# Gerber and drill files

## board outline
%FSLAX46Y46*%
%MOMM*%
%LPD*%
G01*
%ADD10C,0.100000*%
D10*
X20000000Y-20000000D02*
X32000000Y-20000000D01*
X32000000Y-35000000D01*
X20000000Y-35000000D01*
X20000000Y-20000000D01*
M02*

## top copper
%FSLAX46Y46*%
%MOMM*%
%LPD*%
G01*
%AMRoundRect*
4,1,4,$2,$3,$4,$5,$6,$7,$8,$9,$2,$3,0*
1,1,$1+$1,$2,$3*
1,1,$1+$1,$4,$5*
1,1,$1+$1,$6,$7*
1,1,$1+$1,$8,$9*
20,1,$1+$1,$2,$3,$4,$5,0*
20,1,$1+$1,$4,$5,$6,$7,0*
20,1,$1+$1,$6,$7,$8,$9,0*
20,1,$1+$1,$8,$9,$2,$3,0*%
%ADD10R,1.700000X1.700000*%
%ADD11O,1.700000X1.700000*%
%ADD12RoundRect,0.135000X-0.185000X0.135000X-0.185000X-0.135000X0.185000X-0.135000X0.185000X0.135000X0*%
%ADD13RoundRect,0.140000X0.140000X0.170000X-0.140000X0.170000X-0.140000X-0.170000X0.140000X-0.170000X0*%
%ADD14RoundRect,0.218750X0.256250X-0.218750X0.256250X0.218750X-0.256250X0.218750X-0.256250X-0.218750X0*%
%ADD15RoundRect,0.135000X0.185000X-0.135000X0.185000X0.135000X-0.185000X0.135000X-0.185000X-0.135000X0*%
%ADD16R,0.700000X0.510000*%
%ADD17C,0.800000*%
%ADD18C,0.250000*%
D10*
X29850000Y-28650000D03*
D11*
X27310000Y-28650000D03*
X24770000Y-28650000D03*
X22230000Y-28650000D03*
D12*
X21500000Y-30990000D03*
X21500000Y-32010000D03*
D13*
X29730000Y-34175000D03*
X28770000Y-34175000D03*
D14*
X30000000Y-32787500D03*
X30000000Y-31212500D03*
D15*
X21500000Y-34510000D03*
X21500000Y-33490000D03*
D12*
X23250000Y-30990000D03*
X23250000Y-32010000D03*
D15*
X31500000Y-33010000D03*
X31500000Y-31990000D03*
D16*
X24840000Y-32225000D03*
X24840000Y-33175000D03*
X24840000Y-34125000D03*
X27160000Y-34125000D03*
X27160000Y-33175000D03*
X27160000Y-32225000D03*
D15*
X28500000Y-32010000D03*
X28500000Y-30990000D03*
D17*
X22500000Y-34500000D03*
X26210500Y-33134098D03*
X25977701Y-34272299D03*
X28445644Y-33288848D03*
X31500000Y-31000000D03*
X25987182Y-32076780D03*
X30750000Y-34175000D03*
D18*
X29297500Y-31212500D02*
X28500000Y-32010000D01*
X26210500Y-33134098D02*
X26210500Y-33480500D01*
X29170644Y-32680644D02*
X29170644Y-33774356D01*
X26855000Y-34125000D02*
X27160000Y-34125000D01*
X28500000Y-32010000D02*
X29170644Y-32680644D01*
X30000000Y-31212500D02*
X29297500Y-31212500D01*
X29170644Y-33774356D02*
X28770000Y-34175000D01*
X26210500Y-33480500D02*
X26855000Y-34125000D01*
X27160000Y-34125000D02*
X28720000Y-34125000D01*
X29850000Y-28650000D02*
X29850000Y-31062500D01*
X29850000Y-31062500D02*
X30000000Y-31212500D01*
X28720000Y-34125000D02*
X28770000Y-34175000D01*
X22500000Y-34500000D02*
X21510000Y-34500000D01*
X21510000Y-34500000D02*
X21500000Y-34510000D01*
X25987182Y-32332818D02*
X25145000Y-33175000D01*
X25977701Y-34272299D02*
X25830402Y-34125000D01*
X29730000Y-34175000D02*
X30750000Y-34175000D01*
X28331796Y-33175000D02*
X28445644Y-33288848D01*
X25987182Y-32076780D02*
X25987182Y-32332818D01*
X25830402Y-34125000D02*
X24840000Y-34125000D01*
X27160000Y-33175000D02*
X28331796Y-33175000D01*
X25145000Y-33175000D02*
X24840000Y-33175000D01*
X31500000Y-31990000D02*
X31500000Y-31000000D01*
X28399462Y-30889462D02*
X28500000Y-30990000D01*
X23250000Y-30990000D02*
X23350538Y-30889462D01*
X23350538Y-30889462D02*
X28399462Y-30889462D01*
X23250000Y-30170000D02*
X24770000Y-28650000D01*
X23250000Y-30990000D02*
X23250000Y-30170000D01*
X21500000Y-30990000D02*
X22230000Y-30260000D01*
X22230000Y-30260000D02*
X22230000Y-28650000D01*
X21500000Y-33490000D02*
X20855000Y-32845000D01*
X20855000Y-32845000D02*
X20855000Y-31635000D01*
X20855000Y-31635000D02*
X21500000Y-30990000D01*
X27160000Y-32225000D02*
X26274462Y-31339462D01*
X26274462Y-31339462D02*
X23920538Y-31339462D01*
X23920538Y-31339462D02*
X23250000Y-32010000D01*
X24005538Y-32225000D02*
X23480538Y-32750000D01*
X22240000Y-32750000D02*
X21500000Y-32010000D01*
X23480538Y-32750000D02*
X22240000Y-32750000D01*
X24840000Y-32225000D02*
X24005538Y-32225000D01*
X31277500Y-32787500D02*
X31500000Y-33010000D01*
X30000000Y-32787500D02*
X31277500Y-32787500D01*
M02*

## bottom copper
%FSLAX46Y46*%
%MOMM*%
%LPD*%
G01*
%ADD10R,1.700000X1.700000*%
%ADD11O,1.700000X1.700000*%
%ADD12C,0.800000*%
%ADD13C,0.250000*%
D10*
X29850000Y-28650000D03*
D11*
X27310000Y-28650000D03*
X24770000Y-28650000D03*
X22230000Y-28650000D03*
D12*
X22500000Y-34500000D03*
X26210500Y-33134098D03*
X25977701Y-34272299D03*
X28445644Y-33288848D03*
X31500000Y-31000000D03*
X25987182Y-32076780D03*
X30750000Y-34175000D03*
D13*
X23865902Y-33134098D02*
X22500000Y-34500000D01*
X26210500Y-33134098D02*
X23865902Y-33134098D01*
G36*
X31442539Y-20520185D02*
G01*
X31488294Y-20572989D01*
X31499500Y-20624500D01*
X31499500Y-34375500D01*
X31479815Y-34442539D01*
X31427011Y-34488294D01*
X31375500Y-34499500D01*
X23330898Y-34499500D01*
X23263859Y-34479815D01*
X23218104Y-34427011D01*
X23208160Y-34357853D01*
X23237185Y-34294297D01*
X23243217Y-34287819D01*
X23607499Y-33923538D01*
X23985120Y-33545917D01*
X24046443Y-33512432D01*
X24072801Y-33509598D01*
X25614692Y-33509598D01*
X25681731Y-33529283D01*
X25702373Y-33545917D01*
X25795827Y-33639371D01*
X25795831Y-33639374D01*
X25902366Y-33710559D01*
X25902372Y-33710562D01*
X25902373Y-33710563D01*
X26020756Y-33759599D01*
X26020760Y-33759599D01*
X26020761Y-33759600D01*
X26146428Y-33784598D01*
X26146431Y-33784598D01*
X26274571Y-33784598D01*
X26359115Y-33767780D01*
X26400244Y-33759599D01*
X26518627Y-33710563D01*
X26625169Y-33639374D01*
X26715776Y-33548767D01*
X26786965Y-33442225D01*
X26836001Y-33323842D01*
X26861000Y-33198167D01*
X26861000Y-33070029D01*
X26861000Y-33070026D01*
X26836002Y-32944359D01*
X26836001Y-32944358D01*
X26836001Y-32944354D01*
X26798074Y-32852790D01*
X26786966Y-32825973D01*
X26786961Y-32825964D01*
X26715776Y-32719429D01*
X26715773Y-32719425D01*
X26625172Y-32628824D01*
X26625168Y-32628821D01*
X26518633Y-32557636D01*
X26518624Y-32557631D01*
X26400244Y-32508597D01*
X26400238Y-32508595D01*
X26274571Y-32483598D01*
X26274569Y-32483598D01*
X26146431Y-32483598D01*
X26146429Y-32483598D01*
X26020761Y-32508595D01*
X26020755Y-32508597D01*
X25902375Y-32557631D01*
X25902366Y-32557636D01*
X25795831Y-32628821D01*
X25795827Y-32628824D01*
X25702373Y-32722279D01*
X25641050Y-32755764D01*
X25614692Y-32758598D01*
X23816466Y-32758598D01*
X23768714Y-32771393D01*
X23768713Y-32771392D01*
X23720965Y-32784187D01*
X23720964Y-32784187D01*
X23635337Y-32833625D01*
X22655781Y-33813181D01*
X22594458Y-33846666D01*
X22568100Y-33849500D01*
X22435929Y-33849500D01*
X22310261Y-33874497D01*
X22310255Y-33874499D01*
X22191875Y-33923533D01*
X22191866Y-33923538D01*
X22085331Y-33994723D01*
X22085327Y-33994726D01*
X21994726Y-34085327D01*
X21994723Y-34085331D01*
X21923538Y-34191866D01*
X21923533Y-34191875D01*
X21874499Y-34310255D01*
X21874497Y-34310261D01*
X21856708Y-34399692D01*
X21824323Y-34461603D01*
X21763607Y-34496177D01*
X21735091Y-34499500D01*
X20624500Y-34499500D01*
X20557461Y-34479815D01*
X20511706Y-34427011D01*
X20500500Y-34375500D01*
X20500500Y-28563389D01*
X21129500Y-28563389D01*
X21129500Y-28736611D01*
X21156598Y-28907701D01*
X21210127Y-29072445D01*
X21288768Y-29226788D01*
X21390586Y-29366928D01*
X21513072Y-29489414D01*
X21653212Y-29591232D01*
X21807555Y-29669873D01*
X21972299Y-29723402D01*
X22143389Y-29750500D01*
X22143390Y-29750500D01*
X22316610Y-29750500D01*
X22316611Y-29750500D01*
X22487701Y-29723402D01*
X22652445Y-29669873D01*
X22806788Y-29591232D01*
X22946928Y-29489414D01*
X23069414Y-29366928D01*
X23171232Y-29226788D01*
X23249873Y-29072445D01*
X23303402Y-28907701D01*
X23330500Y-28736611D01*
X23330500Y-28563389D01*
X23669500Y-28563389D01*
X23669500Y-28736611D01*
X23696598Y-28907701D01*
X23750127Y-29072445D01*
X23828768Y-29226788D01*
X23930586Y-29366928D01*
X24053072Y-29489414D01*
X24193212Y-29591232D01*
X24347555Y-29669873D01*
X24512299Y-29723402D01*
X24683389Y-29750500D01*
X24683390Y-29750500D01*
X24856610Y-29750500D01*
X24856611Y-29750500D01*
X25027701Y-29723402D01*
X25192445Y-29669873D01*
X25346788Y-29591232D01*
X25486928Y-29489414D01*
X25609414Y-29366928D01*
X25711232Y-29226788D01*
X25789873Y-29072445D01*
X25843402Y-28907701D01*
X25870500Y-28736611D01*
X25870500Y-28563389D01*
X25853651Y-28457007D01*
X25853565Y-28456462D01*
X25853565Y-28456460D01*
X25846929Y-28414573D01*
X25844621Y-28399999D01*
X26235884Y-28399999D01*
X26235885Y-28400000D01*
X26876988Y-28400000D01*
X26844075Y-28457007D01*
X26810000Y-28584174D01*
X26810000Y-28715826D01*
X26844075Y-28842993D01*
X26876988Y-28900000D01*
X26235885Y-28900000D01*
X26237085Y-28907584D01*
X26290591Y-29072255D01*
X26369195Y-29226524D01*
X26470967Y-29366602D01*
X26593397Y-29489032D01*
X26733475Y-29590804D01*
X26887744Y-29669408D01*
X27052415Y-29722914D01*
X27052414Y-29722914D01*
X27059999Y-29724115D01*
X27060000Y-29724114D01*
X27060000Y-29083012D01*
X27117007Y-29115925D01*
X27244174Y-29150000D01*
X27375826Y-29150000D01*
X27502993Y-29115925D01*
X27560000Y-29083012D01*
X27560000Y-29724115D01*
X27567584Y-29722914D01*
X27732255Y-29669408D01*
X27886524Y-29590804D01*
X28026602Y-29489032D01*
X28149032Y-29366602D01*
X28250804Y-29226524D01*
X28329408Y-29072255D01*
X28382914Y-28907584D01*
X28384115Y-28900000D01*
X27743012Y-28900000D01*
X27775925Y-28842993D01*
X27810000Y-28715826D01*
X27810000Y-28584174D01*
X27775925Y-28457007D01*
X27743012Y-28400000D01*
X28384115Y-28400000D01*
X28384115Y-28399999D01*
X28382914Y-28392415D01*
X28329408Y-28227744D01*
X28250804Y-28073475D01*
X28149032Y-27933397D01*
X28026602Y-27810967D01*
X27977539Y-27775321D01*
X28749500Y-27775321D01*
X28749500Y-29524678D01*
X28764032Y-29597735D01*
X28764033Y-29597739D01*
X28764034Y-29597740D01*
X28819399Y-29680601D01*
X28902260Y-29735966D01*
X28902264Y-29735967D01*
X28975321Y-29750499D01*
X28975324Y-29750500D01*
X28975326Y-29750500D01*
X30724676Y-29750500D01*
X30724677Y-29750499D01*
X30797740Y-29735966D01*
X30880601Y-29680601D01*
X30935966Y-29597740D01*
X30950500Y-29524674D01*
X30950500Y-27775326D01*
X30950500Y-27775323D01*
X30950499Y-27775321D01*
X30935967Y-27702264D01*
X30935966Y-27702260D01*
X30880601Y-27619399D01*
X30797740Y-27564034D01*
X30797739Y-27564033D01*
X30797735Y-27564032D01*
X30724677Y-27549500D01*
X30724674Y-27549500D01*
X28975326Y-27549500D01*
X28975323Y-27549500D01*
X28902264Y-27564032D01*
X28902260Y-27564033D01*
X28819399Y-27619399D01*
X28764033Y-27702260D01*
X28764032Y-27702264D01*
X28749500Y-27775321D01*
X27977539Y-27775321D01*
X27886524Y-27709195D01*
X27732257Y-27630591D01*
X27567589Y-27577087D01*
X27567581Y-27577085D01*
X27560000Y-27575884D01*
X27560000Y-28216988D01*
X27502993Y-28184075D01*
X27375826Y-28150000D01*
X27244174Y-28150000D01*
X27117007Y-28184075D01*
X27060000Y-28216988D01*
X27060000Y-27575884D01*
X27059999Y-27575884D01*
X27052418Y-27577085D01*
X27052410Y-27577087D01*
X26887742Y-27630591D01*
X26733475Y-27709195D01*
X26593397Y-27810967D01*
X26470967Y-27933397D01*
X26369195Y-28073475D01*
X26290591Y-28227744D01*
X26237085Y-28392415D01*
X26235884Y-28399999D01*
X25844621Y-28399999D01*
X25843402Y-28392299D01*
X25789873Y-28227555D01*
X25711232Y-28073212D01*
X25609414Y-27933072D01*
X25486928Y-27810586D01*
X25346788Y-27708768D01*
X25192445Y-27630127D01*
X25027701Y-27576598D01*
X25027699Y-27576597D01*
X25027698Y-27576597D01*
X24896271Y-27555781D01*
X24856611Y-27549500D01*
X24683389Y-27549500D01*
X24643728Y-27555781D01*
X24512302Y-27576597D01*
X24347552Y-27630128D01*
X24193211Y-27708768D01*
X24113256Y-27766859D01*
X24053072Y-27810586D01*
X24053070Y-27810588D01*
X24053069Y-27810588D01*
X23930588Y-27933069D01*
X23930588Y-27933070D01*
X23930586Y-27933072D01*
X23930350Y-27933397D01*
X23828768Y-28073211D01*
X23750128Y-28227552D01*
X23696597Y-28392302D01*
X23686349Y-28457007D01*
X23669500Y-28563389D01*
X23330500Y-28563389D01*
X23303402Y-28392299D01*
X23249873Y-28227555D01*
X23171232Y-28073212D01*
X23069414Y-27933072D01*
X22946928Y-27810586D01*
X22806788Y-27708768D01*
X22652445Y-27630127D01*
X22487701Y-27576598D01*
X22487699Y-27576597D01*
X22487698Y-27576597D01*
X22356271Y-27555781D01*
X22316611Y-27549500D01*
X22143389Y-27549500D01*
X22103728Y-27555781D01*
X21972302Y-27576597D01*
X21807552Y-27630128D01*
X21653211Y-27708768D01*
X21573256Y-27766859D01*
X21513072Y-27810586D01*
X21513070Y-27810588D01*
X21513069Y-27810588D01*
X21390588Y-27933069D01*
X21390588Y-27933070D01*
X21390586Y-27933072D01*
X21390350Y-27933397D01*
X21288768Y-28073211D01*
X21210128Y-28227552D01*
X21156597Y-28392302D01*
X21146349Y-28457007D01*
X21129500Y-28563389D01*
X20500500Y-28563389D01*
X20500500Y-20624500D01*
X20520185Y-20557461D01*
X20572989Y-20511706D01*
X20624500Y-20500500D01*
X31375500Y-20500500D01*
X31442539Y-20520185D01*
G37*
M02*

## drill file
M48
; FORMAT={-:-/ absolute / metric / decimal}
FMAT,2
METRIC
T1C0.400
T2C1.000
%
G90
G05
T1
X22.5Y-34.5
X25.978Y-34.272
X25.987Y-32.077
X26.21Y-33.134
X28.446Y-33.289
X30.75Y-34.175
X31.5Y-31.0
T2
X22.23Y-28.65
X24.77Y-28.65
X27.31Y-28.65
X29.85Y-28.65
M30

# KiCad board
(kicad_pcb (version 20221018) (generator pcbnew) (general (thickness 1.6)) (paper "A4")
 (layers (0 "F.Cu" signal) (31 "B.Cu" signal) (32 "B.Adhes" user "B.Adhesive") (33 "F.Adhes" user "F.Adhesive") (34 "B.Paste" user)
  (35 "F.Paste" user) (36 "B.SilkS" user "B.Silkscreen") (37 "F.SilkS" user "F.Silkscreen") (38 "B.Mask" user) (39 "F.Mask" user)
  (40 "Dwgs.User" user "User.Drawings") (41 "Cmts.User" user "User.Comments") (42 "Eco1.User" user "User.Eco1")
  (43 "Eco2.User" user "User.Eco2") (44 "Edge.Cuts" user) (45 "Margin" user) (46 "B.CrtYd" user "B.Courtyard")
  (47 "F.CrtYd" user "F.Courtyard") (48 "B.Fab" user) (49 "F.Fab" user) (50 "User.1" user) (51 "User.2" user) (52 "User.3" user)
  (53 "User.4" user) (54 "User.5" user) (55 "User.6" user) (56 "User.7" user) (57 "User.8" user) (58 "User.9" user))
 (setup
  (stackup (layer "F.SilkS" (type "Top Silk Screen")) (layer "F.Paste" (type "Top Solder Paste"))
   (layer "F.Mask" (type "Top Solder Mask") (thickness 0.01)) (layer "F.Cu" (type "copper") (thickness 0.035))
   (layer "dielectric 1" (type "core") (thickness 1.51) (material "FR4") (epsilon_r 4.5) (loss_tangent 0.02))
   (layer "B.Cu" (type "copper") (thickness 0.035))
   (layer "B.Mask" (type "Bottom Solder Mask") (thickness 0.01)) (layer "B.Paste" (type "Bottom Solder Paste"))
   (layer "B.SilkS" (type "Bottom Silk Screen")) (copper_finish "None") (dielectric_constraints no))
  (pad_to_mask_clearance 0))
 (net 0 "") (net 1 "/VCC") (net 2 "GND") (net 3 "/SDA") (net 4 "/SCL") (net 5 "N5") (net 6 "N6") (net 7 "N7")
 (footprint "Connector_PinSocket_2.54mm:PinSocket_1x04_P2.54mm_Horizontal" (layer "F.Cu") (at 29.85 28.65 -90)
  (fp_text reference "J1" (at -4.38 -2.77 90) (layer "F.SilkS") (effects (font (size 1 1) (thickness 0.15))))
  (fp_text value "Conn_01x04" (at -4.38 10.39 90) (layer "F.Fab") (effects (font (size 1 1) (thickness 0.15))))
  (pad "1" thru_hole rect (at 0 0 270) (size 1.7 1.7) (drill 1) (layers "*.Cu" "*.Mask") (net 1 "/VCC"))
  (pad "2" thru_hole oval (at 0 2.54 270) (size 1.7 1.7) (drill 1) (layers "*.Cu" "*.Mask") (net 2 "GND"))
  (pad "3" thru_hole oval (at 0 5.08 270) (size 1.7 1.7) (drill 1) (layers "*.Cu" "*.Mask") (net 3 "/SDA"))
  (pad "4" thru_hole oval (at 0 7.62 270) (size 1.7 1.7) (drill 1) (layers "*.Cu" "*.Mask") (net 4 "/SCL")))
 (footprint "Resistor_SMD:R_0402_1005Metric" (layer "F.Cu") (at 21.5 31.5 -90)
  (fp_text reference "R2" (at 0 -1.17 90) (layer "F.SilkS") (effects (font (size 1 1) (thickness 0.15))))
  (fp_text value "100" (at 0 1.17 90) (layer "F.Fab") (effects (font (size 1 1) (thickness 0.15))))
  (pad "1" smd roundrect (at -0.51 0 270) (size 0.54 0.64) (layers "F.Cu" "F.Paste" "F.Mask") (roundrect_rratio 0.25) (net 4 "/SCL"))
  (pad "2" smd roundrect (at 0.51 0 270) (size 0.54 0.64) (layers "F.Cu" "F.Paste" "F.Mask") (roundrect_rratio 0.25) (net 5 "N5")))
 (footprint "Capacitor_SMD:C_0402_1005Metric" (layer "F.Cu") (at 29.25 34.175 180)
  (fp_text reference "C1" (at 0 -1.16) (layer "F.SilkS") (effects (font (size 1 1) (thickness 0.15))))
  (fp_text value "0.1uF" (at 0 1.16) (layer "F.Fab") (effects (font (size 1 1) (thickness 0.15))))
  (pad "1" smd roundrect (at -0.48 0 180) (size 0.56 0.62) (layers "F.Cu" "F.Paste" "F.Mask") (roundrect_rratio 0.25) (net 2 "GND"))
  (pad "2" smd roundrect (at 0.48 0 180) (size 0.56 0.62) (layers "F.Cu" "F.Paste" "F.Mask") (roundrect_rratio 0.25) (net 1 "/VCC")))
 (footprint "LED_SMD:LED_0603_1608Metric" (layer "F.Cu") (at 30 32 90)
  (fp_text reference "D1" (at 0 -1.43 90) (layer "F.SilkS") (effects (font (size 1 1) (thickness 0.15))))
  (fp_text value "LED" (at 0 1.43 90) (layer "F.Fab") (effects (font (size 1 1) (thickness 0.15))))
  (pad "1" smd roundrect (at -0.7875 0 90) (size 0.875 0.95) (layers "F.Cu" "F.Paste" "F.Mask") (roundrect_rratio 0.25) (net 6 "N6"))
  (pad "2" smd roundrect (at 0.7875 0 90) (size 0.875 0.95) (layers "F.Cu" "F.Paste" "F.Mask") (roundrect_rratio 0.25) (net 1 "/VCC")))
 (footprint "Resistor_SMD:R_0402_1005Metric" (layer "F.Cu") (at 21.5 34 90)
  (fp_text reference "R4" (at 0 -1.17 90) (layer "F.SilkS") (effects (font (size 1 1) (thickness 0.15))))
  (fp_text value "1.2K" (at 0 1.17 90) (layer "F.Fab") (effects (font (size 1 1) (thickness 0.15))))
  (pad "1" smd roundrect (at -0.51 0 90) (size 0.54 0.64) (layers "F.Cu" "F.Paste" "F.Mask") (roundrect_rratio 0.25) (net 1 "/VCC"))
  (pad "2" smd roundrect (at 0.51 0 90) (size 0.54 0.64) (layers "F.Cu" "F.Paste" "F.Mask") (roundrect_rratio 0.25) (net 4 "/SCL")))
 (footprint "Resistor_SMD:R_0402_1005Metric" (layer "F.Cu") (at 23.25 31.5 -90)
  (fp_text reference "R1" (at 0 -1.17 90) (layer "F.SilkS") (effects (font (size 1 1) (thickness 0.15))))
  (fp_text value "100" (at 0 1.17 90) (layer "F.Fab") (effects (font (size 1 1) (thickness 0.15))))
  (pad "1" smd roundrect (at -0.51 0 270) (size 0.54 0.64) (layers "F.Cu" "F.Paste" "F.Mask") (roundrect_rratio 0.25) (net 3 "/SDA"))
  (pad "2" smd roundrect (at 0.51 0 270) (size 0.54 0.64) (layers "F.Cu" "F.Paste" "F.Mask") (roundrect_rratio 0.25) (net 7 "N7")))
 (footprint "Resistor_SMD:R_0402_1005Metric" (layer "F.Cu") (at 31.5 32.5 90)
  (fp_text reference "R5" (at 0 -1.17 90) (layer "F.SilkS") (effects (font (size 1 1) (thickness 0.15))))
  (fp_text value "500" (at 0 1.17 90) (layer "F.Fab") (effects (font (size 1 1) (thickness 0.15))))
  (pad "1" smd roundrect (at -0.51 0 90) (size 0.54 0.64) (layers "F.Cu" "F.Paste" "F.Mask") (roundrect_rratio 0.25) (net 6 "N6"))
  (pad "2" smd roundrect (at 0.51 0 90) (size 0.54 0.64) (layers "F.Cu" "F.Paste" "F.Mask") (roundrect_rratio 0.25) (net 2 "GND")))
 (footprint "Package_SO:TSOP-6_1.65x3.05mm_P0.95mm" (layer "F.Cu") (at 26 33.175)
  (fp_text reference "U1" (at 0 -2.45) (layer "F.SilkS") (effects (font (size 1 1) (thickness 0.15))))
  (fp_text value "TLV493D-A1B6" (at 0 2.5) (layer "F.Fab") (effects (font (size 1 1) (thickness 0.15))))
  (pad "1" smd rect (at -1.16 -0.95) (size 0.7 0.51) (layers "F.Cu" "F.Paste" "F.Mask") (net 5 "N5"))
  (pad "2" smd rect (at -1.16 0) (size 0.7 0.51) (layers "F.Cu" "F.Paste" "F.Mask") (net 2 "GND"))
  (pad "3" smd rect (at -1.16 0.95) (size 0.7 0.51) (layers "F.Cu" "F.Paste" "F.Mask") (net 2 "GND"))
  (pad "4" smd rect (at 1.16 0.95) (size 0.7 0.51) (layers "F.Cu" "F.Paste" "F.Mask") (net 1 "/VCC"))
  (pad "5" smd rect (at 1.16 0) (size 0.7 0.51) (layers "F.Cu" "F.Paste" "F.Mask") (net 2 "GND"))
  (pad "6" smd rect (at 1.16 -0.95) (size 0.7 0.51) (layers "F.Cu" "F.Paste" "F.Mask") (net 7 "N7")))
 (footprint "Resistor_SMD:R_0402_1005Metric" (layer "F.Cu") (at 28.5 31.5 90)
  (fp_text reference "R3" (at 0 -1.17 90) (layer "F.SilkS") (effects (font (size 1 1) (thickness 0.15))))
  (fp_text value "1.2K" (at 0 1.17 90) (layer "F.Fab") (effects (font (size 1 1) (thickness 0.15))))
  (pad "1" smd roundrect (at -0.51 0 90) (size 0.54 0.64) (layers "F.Cu" "F.Paste" "F.Mask") (roundrect_rratio 0.25) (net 1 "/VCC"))
  (pad "2" smd roundrect (at 0.51 0 90) (size 0.54 0.64) (layers "F.Cu" "F.Paste" "F.Mask") (roundrect_rratio 0.25) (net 3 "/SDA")))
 (gr_rect (start 20 20) (end 32 35) (stroke (width 0.1) (type default)) (fill none) (layer "Edge.Cuts"))
 (segment (start 29.2975 31.2125) (end 28.5 32.01) (width 0.25) (layer "F.Cu") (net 1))
 (segment (start 26.2105 33.134098) (end 26.2105 33.4805) (width 0.25) (layer "F.Cu") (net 1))
 (segment (start 29.170644 32.680644) (end 29.170644 33.774356) (width 0.25) (layer "F.Cu") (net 1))
 (segment (start 26.855 34.125) (end 27.16 34.125) (width 0.25) (layer "F.Cu") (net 1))
 (segment (start 28.5 32.01) (end 29.170644 32.680644) (width 0.25) (layer "F.Cu") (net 1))
 (segment (start 30 31.2125) (end 29.2975 31.2125) (width 0.25) (layer "F.Cu") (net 1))
 (segment (start 29.170644 33.774356) (end 28.77 34.175) (width 0.25) (layer "F.Cu") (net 1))
 (segment (start 26.2105 33.4805) (end 26.855 34.125) (width 0.25) (layer "F.Cu") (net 1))
 (segment (start 27.16 34.125) (end 28.72 34.125) (width 0.25) (layer "F.Cu") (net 1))
 (segment (start 29.85 28.65) (end 29.85 31.0625) (width 0.25) (layer "F.Cu") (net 1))
 (segment (start 29.85 31.0625) (end 30 31.2125) (width 0.25) (layer "F.Cu") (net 1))
 (segment (start 28.72 34.125) (end 28.77 34.175) (width 0.25) (layer "F.Cu") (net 1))
 (segment (start 22.5 34.5) (end 21.51 34.5) (width 0.25) (layer "F.Cu") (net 1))
 (segment (start 21.51 34.5) (end 21.5 34.51) (width 0.25) (layer "F.Cu") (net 1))
 (via (at 22.5 34.5) (size 0.8) (drill 0.4) (layers "F.Cu" "B.Cu") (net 1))
 (via (at 26.2105 33.134098) (size 0.8) (drill 0.4) (layers "F.Cu" "B.Cu") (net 1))
 (segment (start 23.865902 33.134098) (end 22.5 34.5) (width 0.25) (layer "B.Cu") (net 1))
 (segment (start 26.2105 33.134098) (end 23.865902 33.134098) (width 0.25) (layer "B.Cu") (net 1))
 (segment (start 25.987182 32.332818) (end 25.145 33.175) (width 0.25) (layer "F.Cu") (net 2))
 (segment (start 25.977701 34.272299) (end 25.830402 34.125) (width 0.25) (layer "F.Cu") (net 2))
 (segment (start 29.73 34.175) (end 30.75 34.175) (width 0.25) (layer "F.Cu") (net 2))
 (segment (start 28.331796 33.175) (end 28.445644 33.288848) (width 0.25) (layer "F.Cu") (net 2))
 (segment (start 25.987182 32.07678) (end 25.987182 32.332818) (width 0.25) (layer "F.Cu") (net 2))
 (segment (start 25.830402 34.125) (end 24.84 34.125) (width 0.25) (layer "F.Cu") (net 2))
 (segment (start 27.16 33.175) (end 28.331796 33.175) (width 0.25) (layer "F.Cu") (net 2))
 (segment (start 25.145 33.175) (end 24.84 33.175) (width 0.25) (layer "F.Cu") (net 2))
 (segment (start 31.5 31.99) (end 31.5 31) (width 0.25) (layer "F.Cu") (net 2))
 (via (at 25.977701 34.272299) (size 0.8) (drill 0.4) (layers "F.Cu" "B.Cu") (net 2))
 (via (at 28.445644 33.288848) (size 0.8) (drill 0.4) (layers "F.Cu" "B.Cu") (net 2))
 (via (at 31.5 31) (size 0.8) (drill 0.4) (layers "F.Cu" "B.Cu") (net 2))
 (via (at 25.987182 32.07678) (size 0.8) (drill 0.4) (layers "F.Cu" "B.Cu") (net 2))
 (via (at 30.75 34.175) (size 0.8) (drill 0.4) (layers "F.Cu" "B.Cu") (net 2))
 (segment (start 28.399462 30.889462) (end 28.5 30.99) (width 0.25) (layer "F.Cu") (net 3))
 (segment (start 23.25 30.99) (end 23.350538 30.889462) (width 0.25) (layer "F.Cu") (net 3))
 (segment (start 23.350538 30.889462) (end 28.399462 30.889462) (width 0.25) (layer "F.Cu") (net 3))
 (segment (start 23.25 30.17) (end 24.77 28.65) (width 0.25) (layer "F.Cu") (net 3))
 (segment (start 23.25 30.99) (end 23.25 30.17) (width 0.25) (layer "F.Cu") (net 3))
 (segment (start 21.5 30.99) (end 22.23 30.26) (width 0.25) (layer "F.Cu") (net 4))
 (segment (start 22.23 30.26) (end 22.23 28.65) (width 0.25) (layer "F.Cu") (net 4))
 (segment (start 21.5 33.49) (end 20.855 32.845) (width 0.25) (layer "F.Cu") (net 4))
 (segment (start 20.855 32.845) (end 20.855 31.635) (width 0.25) (layer "F.Cu") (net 4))
 (segment (start 20.855 31.635) (end 21.5 30.99) (width 0.25) (layer "F.Cu") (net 4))
 (segment (start 27.16 32.225) (end 26.274462 31.339462) (width 0.25) (layer "F.Cu") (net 7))
 (segment (start 26.274462 31.339462) (end 23.920538 31.339462) (width 0.25) (layer "F.Cu") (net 7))
 (segment (start 23.920538 31.339462) (end 23.25 32.01) (width 0.25) (layer "F.Cu") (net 7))
 (segment (start 24.005538 32.225) (end 23.480538 32.75) (width 0.25) (layer "F.Cu") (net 5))
 (segment (start 22.24 32.75) (end 21.5 32.01) (width 0.25) (layer "F.Cu") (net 5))
 (segment (start 23.480538 32.75) (end 22.24 32.75) (width 0.25) (layer "F.Cu") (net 5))
 (segment (start 24.84 32.225) (end 24.005538 32.225) (width 0.25) (layer "F.Cu") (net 5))
 (segment (start 31.2775 32.7875) (end 31.5 33.01) (width 0.25) (layer "F.Cu") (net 6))
 (segment (start 30 32.7875) (end 31.2775 32.7875) (width 0.25) (layer "F.Cu") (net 6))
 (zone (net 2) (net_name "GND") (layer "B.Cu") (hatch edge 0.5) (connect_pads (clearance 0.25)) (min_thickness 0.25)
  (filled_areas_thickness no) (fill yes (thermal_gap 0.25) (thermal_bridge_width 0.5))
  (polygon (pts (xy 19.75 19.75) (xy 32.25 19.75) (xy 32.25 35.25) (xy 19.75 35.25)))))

